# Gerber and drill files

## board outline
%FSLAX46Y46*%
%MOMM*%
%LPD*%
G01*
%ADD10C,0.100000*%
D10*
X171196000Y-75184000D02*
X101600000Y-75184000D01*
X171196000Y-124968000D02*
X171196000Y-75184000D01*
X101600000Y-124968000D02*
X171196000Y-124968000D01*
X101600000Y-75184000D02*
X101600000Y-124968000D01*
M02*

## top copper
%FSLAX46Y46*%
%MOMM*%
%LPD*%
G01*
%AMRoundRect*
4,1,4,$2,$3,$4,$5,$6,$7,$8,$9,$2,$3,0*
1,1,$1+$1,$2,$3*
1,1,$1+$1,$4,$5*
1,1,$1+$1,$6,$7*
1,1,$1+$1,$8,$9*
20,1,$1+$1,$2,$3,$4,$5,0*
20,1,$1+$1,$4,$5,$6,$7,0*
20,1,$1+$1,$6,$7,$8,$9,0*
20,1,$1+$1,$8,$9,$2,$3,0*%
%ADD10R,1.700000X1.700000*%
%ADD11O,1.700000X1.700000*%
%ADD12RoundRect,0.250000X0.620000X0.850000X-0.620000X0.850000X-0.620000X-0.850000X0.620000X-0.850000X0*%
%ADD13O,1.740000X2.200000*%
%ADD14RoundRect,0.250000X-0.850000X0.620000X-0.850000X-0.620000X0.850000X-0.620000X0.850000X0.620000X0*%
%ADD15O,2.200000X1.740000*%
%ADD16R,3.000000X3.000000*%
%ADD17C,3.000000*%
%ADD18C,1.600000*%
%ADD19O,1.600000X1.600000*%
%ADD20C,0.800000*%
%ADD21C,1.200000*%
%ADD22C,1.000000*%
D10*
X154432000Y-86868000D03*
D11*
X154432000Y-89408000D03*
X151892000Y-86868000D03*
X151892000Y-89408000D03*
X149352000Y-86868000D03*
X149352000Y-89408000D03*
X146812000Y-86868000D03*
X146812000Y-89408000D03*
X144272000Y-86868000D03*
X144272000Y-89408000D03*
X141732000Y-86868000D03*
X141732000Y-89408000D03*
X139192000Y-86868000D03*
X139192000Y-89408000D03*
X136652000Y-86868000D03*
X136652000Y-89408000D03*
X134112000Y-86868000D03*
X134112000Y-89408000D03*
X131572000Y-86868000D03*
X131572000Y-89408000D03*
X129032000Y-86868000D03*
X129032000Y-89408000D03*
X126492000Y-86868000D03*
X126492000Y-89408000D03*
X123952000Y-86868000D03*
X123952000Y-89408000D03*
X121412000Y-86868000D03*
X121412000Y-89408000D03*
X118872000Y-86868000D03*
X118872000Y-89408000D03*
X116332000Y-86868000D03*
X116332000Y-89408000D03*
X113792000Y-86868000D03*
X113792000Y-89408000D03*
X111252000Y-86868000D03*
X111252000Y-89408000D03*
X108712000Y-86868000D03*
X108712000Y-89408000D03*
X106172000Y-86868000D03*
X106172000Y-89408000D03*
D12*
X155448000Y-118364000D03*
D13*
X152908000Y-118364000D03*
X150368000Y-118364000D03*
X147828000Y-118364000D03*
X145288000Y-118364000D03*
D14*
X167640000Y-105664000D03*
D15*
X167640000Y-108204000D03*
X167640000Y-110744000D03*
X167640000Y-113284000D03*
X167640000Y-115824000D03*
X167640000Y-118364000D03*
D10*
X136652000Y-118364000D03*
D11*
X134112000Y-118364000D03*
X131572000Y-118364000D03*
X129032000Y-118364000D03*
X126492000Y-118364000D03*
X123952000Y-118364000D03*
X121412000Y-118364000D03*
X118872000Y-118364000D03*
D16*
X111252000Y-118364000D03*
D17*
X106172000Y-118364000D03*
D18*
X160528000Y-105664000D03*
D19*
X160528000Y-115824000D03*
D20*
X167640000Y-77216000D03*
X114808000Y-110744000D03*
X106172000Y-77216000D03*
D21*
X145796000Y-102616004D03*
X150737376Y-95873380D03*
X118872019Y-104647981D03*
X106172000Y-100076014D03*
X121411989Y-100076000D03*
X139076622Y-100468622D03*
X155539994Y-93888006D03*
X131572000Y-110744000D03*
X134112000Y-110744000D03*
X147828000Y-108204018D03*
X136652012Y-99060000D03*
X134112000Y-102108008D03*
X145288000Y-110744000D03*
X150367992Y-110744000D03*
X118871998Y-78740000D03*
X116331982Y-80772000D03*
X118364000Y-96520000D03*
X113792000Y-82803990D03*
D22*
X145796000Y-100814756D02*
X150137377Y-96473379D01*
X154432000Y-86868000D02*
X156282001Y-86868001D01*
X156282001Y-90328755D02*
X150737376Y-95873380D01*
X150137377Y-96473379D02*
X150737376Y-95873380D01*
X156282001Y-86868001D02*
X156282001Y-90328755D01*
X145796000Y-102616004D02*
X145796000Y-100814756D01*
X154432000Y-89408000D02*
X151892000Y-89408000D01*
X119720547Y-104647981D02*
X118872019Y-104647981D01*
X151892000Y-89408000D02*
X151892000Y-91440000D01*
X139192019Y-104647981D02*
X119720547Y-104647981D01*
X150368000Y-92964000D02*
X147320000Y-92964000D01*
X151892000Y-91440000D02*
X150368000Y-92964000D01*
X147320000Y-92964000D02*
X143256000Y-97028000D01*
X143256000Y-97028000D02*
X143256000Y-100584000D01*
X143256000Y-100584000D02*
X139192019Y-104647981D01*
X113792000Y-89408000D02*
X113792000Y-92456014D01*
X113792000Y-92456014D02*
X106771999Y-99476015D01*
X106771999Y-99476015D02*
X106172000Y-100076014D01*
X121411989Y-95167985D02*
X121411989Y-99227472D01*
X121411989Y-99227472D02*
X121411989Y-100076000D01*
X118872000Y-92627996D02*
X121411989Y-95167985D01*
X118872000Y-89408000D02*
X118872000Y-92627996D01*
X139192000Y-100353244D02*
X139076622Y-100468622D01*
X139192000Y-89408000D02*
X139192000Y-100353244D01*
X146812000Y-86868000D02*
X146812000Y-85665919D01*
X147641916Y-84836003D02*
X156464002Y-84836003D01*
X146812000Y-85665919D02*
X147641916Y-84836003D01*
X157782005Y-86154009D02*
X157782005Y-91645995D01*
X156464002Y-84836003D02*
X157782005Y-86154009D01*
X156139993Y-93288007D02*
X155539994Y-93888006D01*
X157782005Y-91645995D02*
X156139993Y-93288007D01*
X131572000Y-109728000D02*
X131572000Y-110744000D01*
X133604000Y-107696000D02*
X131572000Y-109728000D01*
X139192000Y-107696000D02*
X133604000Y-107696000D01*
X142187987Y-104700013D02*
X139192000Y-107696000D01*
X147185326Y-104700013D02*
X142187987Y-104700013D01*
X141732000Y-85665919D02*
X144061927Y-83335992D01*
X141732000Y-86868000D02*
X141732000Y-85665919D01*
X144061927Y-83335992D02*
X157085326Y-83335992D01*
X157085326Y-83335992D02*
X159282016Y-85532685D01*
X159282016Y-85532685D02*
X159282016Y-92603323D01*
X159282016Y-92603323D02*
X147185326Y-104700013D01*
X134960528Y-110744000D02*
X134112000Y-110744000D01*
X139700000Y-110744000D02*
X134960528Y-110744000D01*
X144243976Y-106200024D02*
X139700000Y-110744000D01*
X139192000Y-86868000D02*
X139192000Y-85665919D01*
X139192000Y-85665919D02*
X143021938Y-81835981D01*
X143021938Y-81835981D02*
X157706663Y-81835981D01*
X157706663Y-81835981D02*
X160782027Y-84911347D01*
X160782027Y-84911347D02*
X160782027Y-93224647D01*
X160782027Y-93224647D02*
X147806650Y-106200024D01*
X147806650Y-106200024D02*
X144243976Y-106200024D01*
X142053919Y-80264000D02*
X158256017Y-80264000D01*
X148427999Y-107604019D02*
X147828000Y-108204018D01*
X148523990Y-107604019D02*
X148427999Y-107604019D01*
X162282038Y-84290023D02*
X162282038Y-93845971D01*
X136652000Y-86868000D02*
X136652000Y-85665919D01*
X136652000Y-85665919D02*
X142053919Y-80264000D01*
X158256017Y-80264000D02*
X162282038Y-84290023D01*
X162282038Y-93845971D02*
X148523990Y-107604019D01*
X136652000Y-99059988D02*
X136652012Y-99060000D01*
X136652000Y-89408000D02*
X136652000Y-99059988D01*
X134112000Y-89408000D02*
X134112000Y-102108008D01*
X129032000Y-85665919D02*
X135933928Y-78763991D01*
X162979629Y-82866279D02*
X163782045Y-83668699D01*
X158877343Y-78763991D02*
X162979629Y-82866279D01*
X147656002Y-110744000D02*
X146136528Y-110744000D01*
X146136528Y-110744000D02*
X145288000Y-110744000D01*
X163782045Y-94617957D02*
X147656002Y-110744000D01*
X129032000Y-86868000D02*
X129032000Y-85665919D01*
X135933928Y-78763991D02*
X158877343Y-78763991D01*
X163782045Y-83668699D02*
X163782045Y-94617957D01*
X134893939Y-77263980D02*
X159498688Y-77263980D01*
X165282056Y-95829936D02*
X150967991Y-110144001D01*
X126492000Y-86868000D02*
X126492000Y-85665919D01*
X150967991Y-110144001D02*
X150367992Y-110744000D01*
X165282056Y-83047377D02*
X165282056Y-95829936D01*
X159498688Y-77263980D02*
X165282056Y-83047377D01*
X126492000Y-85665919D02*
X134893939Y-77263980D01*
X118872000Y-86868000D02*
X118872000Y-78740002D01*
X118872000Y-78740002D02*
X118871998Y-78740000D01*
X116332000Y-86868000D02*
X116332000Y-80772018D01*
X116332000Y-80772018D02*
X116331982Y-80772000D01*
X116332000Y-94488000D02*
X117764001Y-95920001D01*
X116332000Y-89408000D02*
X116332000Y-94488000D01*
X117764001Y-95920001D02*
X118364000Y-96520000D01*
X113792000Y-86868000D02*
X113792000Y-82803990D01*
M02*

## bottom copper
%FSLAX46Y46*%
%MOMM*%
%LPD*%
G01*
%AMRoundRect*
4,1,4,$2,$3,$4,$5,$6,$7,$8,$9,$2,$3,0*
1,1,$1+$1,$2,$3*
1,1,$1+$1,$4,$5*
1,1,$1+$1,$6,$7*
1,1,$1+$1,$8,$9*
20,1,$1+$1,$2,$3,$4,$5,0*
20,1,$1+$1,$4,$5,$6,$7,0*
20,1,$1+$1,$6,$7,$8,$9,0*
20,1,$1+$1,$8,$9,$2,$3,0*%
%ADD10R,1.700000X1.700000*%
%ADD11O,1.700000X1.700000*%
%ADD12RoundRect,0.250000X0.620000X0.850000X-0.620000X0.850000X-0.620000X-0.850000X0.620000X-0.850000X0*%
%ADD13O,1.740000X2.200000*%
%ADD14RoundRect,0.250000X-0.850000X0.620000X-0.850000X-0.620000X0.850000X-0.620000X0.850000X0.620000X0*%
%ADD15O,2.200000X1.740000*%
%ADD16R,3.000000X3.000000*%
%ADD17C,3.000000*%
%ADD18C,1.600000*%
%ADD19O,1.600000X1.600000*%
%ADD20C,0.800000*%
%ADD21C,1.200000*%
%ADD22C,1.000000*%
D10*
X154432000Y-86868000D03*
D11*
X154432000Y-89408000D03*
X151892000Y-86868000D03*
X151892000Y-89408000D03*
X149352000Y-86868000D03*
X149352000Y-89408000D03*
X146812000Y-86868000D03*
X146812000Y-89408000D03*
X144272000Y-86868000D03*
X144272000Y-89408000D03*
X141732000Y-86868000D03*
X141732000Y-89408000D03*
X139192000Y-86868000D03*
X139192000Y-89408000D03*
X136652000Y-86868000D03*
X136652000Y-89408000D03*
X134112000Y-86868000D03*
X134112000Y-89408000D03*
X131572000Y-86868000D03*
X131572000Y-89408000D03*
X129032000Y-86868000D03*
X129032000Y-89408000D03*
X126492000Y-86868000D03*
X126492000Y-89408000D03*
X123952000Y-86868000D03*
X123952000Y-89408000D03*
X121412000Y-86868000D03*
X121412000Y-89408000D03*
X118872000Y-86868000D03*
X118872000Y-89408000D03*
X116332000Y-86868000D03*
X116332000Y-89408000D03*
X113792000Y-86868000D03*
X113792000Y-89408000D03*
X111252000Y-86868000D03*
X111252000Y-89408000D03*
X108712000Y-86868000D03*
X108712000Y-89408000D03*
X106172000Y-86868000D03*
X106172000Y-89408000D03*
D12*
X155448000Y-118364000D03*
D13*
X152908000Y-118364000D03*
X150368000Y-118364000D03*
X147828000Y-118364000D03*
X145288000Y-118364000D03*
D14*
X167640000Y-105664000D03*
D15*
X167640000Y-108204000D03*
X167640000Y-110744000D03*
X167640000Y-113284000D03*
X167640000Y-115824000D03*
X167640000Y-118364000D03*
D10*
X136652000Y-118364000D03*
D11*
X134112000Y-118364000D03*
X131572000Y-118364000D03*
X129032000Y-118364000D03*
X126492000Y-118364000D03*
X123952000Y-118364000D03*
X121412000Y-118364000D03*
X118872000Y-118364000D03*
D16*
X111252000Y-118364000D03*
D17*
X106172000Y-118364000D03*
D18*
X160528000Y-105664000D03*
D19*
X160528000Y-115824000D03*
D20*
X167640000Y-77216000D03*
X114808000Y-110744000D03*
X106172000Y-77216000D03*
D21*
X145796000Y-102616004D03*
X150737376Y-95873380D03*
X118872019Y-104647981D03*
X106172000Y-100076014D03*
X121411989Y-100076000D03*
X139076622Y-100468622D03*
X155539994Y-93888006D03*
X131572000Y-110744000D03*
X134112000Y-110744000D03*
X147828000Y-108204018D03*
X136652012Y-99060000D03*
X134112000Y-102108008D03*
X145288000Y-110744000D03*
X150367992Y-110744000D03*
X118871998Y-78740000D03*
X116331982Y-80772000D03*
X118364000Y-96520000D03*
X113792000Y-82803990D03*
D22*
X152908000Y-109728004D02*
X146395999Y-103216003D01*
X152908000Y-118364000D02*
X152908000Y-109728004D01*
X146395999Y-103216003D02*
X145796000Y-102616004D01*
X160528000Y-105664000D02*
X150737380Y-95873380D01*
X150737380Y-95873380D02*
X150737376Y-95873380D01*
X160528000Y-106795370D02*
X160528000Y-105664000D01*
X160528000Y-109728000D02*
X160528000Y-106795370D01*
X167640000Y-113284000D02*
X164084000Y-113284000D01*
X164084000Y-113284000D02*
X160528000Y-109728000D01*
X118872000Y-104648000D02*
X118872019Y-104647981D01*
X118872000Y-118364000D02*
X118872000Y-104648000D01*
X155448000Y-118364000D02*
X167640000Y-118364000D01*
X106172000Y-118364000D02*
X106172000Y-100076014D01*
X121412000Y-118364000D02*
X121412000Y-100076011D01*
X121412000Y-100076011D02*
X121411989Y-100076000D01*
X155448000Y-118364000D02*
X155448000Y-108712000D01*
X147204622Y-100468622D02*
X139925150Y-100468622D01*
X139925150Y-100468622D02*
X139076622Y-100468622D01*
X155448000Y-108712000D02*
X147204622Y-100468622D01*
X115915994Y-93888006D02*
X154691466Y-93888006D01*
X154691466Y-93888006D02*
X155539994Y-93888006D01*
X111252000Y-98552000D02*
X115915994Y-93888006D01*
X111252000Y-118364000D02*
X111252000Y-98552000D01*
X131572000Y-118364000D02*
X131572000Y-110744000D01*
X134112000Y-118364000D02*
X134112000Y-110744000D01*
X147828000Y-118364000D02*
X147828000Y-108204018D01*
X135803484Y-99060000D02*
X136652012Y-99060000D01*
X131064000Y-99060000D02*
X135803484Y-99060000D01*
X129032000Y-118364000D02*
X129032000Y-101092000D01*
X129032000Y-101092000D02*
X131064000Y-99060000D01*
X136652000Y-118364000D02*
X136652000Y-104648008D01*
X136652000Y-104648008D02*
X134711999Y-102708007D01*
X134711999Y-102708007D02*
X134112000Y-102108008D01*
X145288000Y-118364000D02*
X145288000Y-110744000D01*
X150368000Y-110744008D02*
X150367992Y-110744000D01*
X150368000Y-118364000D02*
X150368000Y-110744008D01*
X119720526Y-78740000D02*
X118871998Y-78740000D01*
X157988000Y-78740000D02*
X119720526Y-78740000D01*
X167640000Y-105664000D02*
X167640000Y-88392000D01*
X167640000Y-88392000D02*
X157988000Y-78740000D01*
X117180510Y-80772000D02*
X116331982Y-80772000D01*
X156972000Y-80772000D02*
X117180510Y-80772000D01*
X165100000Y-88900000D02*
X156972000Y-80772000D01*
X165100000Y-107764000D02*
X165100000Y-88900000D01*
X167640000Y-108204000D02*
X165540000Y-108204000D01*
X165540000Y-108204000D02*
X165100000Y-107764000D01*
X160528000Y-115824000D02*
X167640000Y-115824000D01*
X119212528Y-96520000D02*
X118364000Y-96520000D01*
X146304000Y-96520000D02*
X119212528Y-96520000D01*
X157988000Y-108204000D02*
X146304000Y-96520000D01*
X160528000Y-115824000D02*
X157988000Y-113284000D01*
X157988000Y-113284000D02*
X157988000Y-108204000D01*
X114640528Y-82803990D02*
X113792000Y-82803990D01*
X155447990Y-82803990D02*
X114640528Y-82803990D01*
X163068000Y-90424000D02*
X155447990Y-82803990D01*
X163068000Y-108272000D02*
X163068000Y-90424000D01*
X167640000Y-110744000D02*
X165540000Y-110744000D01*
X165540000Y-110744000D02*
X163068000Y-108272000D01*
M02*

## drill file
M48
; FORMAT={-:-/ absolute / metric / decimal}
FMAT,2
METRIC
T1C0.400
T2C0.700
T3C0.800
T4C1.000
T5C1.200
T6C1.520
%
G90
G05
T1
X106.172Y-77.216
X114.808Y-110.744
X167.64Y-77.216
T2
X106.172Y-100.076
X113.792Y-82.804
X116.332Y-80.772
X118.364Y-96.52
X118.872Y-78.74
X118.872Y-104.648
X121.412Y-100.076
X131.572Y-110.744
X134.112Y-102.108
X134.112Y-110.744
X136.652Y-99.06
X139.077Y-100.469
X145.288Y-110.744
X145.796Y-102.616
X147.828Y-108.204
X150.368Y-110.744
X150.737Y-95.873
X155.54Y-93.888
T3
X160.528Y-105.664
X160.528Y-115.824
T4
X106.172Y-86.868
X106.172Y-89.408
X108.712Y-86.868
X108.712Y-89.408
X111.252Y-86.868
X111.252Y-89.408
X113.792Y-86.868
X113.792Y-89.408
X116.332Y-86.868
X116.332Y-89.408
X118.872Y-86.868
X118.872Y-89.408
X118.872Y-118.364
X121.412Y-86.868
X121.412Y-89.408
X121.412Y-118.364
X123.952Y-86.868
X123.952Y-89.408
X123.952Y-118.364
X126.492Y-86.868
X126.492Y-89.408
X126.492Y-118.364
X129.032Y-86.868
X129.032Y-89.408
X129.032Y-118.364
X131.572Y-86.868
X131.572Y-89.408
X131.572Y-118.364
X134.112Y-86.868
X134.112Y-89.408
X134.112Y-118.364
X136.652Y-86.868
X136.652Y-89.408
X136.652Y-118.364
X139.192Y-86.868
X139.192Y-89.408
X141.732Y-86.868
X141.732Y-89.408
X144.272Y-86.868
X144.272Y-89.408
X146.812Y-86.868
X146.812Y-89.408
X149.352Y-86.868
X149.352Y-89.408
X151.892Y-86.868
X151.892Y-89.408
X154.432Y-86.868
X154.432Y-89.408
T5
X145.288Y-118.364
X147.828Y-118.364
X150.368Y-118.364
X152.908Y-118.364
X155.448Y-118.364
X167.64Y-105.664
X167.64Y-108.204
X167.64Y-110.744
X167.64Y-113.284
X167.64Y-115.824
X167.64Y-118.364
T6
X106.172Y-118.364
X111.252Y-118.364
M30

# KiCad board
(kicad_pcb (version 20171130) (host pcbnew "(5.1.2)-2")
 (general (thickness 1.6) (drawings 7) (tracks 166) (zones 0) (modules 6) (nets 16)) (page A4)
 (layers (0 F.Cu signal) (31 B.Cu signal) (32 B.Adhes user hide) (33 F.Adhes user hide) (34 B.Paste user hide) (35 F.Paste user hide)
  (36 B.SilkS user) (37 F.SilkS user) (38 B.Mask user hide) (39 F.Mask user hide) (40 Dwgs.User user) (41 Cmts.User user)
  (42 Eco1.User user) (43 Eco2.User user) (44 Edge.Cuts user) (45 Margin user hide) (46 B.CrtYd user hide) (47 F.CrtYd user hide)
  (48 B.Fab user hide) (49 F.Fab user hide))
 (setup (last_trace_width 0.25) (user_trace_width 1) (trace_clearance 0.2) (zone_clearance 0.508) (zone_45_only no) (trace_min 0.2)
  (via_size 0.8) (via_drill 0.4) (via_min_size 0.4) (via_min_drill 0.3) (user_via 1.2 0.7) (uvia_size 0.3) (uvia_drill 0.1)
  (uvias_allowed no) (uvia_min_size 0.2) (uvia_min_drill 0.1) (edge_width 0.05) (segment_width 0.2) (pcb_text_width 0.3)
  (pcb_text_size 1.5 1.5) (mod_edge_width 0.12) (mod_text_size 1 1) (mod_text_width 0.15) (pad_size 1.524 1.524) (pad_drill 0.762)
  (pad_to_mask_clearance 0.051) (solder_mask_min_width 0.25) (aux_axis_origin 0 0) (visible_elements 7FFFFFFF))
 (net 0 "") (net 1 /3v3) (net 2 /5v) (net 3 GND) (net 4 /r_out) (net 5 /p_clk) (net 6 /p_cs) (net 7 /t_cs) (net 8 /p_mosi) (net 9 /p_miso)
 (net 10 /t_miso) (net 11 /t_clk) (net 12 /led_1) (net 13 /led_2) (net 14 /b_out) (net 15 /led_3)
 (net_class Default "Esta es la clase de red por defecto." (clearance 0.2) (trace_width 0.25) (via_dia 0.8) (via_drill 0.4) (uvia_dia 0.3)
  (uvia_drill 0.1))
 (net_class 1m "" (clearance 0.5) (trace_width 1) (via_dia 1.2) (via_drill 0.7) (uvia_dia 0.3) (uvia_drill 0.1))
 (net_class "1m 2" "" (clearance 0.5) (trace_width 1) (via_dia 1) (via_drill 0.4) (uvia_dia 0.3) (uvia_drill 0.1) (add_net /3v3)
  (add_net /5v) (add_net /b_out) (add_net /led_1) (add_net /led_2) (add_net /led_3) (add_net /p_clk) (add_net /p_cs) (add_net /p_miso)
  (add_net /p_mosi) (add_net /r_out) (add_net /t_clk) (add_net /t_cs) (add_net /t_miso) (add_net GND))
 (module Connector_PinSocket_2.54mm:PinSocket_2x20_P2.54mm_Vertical (layer B.Cu) (at 154.432 86.868 90)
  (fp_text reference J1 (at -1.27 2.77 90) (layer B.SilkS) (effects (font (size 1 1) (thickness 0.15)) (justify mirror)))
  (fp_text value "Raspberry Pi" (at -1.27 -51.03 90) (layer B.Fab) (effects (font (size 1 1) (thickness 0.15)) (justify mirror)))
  (pad 1 thru_hole rect (at 0 0 90) (size 1.7 1.7) (drill 1) (layers *.Cu *.Mask) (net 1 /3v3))
  (pad 2 thru_hole oval (at -2.54 0 90) (size 1.7 1.7) (drill 1) (layers *.Cu *.Mask) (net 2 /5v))
  (pad 3 thru_hole oval (at 0 -2.54 90) (size 1.7 1.7) (drill 1) (layers *.Cu *.Mask))
  (pad 4 thru_hole oval (at -2.54 -2.54 90) (size 1.7 1.7) (drill 1) (layers *.Cu *.Mask) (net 2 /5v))
  (pad 5 thru_hole oval (at 0 -5.08 90) (size 1.7 1.7) (drill 1) (layers *.Cu *.Mask))
  (pad 6 thru_hole oval (at -2.54 -5.08 90) (size 1.7 1.7) (drill 1) (layers *.Cu *.Mask) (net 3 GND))
  (pad 7 thru_hole oval (at 0 -7.62 90) (size 1.7 1.7) (drill 1) (layers *.Cu *.Mask) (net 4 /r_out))
  (pad 8 thru_hole oval (at -2.54 -7.62 90) (size 1.7 1.7) (drill 1) (layers *.Cu *.Mask))
  (pad 9 thru_hole oval (at 0 -10.16 90) (size 1.7 1.7) (drill 1) (layers *.Cu *.Mask))
  (pad 10 thru_hole oval (at -2.54 -10.16 90) (size 1.7 1.7) (drill 1) (layers *.Cu *.Mask))
  (pad 11 thru_hole oval (at 0 -12.7 90) (size 1.7 1.7) (drill 1) (layers *.Cu *.Mask) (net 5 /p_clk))
  (pad 12 thru_hole oval (at -2.54 -12.7 90) (size 1.7 1.7) (drill 1) (layers *.Cu *.Mask))
  (pad 13 thru_hole oval (at 0 -15.24 90) (size 1.7 1.7) (drill 1) (layers *.Cu *.Mask) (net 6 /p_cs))
  (pad 14 thru_hole oval (at -2.54 -15.24 90) (size 1.7 1.7) (drill 1) (layers *.Cu *.Mask) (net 3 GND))
  (pad 15 thru_hole oval (at 0 -17.78 90) (size 1.7 1.7) (drill 1) (layers *.Cu *.Mask) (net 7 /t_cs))
  (pad 16 thru_hole oval (at -2.54 -17.78 90) (size 1.7 1.7) (drill 1) (layers *.Cu *.Mask) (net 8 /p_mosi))
  (pad 17 thru_hole oval (at 0 -20.32 90) (size 1.7 1.7) (drill 1) (layers *.Cu *.Mask))
  (pad 18 thru_hole oval (at -2.54 -20.32 90) (size 1.7 1.7) (drill 1) (layers *.Cu *.Mask) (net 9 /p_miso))
  (pad 19 thru_hole oval (at 0 -22.86 90) (size 1.7 1.7) (drill 1) (layers *.Cu *.Mask))
  (pad 20 thru_hole oval (at -2.54 -22.86 90) (size 1.7 1.7) (drill 1) (layers *.Cu *.Mask) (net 3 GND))
  (pad 21 thru_hole oval (at 0 -25.4 90) (size 1.7 1.7) (drill 1) (layers *.Cu *.Mask) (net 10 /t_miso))
  (pad 22 thru_hole oval (at -2.54 -25.4 90) (size 1.7 1.7) (drill 1) (layers *.Cu *.Mask))
  (pad 23 thru_hole oval (at 0 -27.94 90) (size 1.7 1.7) (drill 1) (layers *.Cu *.Mask) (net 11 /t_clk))
  (pad 24 thru_hole oval (at -2.54 -27.94 90) (size 1.7 1.7) (drill 1) (layers *.Cu *.Mask))
  (pad 25 thru_hole oval (at 0 -30.48 90) (size 1.7 1.7) (drill 1) (layers *.Cu *.Mask))
  (pad 26 thru_hole oval (at -2.54 -30.48 90) (size 1.7 1.7) (drill 1) (layers *.Cu *.Mask))
  (pad 27 thru_hole oval (at 0 -33.02 90) (size 1.7 1.7) (drill 1) (layers *.Cu *.Mask))
  (pad 28 thru_hole oval (at -2.54 -33.02 90) (size 1.7 1.7) (drill 1) (layers *.Cu *.Mask))
  (pad 29 thru_hole oval (at 0 -35.56 90) (size 1.7 1.7) (drill 1) (layers *.Cu *.Mask) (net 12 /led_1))
  (pad 30 thru_hole oval (at -2.54 -35.56 90) (size 1.7 1.7) (drill 1) (layers *.Cu *.Mask) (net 3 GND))
  (pad 31 thru_hole oval (at 0 -38.1 90) (size 1.7 1.7) (drill 1) (layers *.Cu *.Mask) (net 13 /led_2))
  (pad 32 thru_hole oval (at -2.54 -38.1 90) (size 1.7 1.7) (drill 1) (layers *.Cu *.Mask) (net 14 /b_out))
  (pad 33 thru_hole oval (at 0 -40.64 90) (size 1.7 1.7) (drill 1) (layers *.Cu *.Mask) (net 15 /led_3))
  (pad 34 thru_hole oval (at -2.54 -40.64 90) (size 1.7 1.7) (drill 1) (layers *.Cu *.Mask) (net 3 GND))
  (pad 35 thru_hole oval (at 0 -43.18 90) (size 1.7 1.7) (drill 1) (layers *.Cu *.Mask))
  (pad 36 thru_hole oval (at -2.54 -43.18 90) (size 1.7 1.7) (drill 1) (layers *.Cu *.Mask))
  (pad 37 thru_hole oval (at 0 -45.72 90) (size 1.7 1.7) (drill 1) (layers *.Cu *.Mask))
  (pad 38 thru_hole oval (at -2.54 -45.72 90) (size 1.7 1.7) (drill 1) (layers *.Cu *.Mask))
  (pad 39 thru_hole oval (at 0 -48.26 90) (size 1.7 1.7) (drill 1) (layers *.Cu *.Mask))
  (pad 40 thru_hole oval (at -2.54 -48.26 90) (size 1.7 1.7) (drill 1) (layers *.Cu *.Mask)))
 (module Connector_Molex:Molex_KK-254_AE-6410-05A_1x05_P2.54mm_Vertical (layer F.Cu) (at 155.448 118.364 180)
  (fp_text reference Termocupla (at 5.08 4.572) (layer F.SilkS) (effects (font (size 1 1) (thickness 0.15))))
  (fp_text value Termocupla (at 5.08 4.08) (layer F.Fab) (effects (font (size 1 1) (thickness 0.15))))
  (pad 1 thru_hole roundrect (at 0 0 180) (size 1.74 2.2) (drill 1.2) (layers *.Cu *.Mask) (roundrect_rratio 0.143678) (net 3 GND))
  (pad 2 thru_hole oval (at 2.54 0 180) (size 1.74 2.2) (drill 1.2) (layers *.Cu *.Mask) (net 1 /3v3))
  (pad 3 thru_hole oval (at 5.08 0 180) (size 1.74 2.2) (drill 1.2) (layers *.Cu *.Mask) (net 11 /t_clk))
  (pad 4 thru_hole oval (at 7.62 0 180) (size 1.74 2.2) (drill 1.2) (layers *.Cu *.Mask) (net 7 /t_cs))
  (pad 5 thru_hole oval (at 10.16 0 180) (size 1.74 2.2) (drill 1.2) (layers *.Cu *.Mask) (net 10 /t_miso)))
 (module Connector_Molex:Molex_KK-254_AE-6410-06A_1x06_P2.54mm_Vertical (layer F.Cu) (at 167.64 105.664 270)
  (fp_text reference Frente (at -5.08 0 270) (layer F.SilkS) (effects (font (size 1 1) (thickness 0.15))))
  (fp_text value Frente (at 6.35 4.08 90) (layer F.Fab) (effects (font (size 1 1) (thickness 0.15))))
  (pad 1 thru_hole roundrect (at 0 0 270) (size 1.74 2.2) (drill 1.2) (layers *.Cu *.Mask) (roundrect_rratio 0.143678) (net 12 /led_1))
  (pad 2 thru_hole oval (at 2.54 0 270) (size 1.74 2.2) (drill 1.2) (layers *.Cu *.Mask) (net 13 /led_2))
  (pad 3 thru_hole oval (at 5.08 0 270) (size 1.74 2.2) (drill 1.2) (layers *.Cu *.Mask) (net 15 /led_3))
  (pad 4 thru_hole oval (at 7.62 0 270) (size 1.74 2.2) (drill 1.2) (layers *.Cu *.Mask) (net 1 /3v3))
  (pad 5 thru_hole oval (at 10.16 0 270) (size 1.74 2.2) (drill 1.2) (layers *.Cu *.Mask) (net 14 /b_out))
  (pad 6 thru_hole oval (at 12.7 0 270) (size 1.74 2.2) (drill 1.2) (layers *.Cu *.Mask) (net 3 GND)))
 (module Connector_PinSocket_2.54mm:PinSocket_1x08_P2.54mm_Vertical (layer F.Cu) (at 136.652 118.364 270)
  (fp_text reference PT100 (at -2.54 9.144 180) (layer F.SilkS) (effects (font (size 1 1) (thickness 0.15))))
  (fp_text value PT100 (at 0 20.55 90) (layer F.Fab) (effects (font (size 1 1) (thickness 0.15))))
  (pad 1 thru_hole rect (at 0 0 270) (size 1.7 1.7) (drill 1) (layers *.Cu *.Mask) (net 9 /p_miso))
  (pad 2 thru_hole oval (at 0 2.54 270) (size 1.7 1.7) (drill 1) (layers *.Cu *.Mask) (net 6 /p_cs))
  (pad 3 thru_hole oval (at 0 5.08 270) (size 1.7 1.7) (drill 1) (layers *.Cu *.Mask) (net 5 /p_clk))
  (pad 4 thru_hole oval (at 0 7.62 270) (size 1.7 1.7) (drill 1) (layers *.Cu *.Mask) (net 8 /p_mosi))
  (pad 5 thru_hole oval (at 0 10.16 270) (size 1.7 1.7) (drill 1) (layers *.Cu *.Mask))
  (pad 6 thru_hole oval (at 0 12.7 270) (size 1.7 1.7) (drill 1) (layers *.Cu *.Mask))
  (pad 7 thru_hole oval (at 0 15.24 270) (size 1.7 1.7) (drill 1) (layers *.Cu *.Mask) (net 3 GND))
  (pad 8 thru_hole oval (at 0 17.78 270) (size 1.7 1.7) (drill 1) (layers *.Cu *.Mask) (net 2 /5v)))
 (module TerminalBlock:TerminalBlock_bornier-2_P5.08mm (layer F.Cu) (at 111.252 118.364 180)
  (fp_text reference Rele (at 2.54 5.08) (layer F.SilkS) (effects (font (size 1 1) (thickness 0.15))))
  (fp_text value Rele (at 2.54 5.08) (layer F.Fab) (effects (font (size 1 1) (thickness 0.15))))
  (pad 1 thru_hole rect (at 0 0 180) (size 3 3) (drill 1.52) (layers *.Cu *.Mask) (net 4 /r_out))
  (pad 2 thru_hole circle (at 5.08 0 180) (size 3 3) (drill 1.52) (layers *.Cu *.Mask) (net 3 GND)))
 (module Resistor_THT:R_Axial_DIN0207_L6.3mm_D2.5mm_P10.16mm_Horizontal (layer F.Cu) (at 160.528 105.664 270)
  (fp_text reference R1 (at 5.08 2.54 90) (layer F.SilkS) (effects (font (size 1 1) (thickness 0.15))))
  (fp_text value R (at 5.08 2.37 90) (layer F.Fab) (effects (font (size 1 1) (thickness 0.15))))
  (pad 1 thru_hole circle (at 0 0 270) (size 1.6 1.6) (drill 0.8) (layers *.Cu *.Mask) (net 1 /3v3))
  (pad 2 thru_hole oval (at 10.16 0 270) (size 1.6 1.6) (drill 0.8) (layers *.Cu *.Mask) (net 14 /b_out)))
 (gr_line (start 171.196 75.184) (end 101.6 75.184) (layer Edge.Cuts) (width 0.1))
 (gr_line (start 171.196 124.968) (end 171.196 75.184) (layer Edge.Cuts) (width 0.1))
 (gr_line (start 101.6 124.968) (end 171.196 124.968) (layer Edge.Cuts) (width 0.1))
 (gr_line (start 101.6 75.184) (end 101.6 124.968) (layer Edge.Cuts) (width 0.1))
 (via (at 167.64 77.216) (size 0.8) (drill 0.4) (layers F.Cu B.Cu) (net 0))
 (via (at 114.808 110.744) (size 0.8) (drill 0.4) (layers F.Cu B.Cu) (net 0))
 (via (at 106.172 77.216) (size 0.8) (drill 0.4) (layers F.Cu B.Cu) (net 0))
 (segment (start 152.908 109.728004) (end 146.395999 103.216003) (width 1) (layer B.Cu) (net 1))
 (segment (start 152.908 118.364) (end 152.908 109.728004) (width 1) (layer B.Cu) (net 1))
 (via (at 145.796 102.616004) (size 1.2) (drill 0.7) (layers F.Cu B.Cu) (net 1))
 (segment (start 146.395999 103.216003) (end 145.796 102.616004) (width 1) (layer B.Cu) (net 1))
 (via (at 150.737376 95.87338) (size 1.2) (drill 0.7) (layers F.Cu B.Cu) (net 1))
 (segment (start 145.796 100.814756) (end 150.137377 96.473379) (width 1) (layer F.Cu) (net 1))
 (segment (start 160.528 105.664) (end 150.73738 95.87338) (width 1) (layer B.Cu) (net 1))
 (segment (start 154.432 86.868) (end 156.282001 86.868001) (width 1) (layer F.Cu) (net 1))
 (segment (start 156.282001 90.328755) (end 150.737376 95.87338) (width 1) (layer F.Cu) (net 1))
 (segment (start 150.137377 96.473379) (end 150.737376 95.87338) (width 1) (layer F.Cu) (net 1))
 (segment (start 156.282001 86.868001) (end 156.282001 90.328755) (width 1) (layer F.Cu) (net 1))
 (segment (start 145.796 102.616004) (end 145.796 100.814756) (width 1) (layer F.Cu) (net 1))
 (segment (start 150.73738 95.87338) (end 150.737376 95.87338) (width 1) (layer B.Cu) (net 1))
 (segment (start 160.528 106.79537) (end 160.528 105.664) (width 1) (layer B.Cu) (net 1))
 (segment (start 160.528 109.728) (end 160.528 106.79537) (width 1) (layer B.Cu) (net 1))
 (segment (start 167.64 113.284) (end 164.084 113.284) (width 1) (layer B.Cu) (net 1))
 (segment (start 164.084 113.284) (end 160.528 109.728) (width 1) (layer B.Cu) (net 1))
 (segment (start 154.432 89.408) (end 151.892 89.408) (width 1) (layer F.Cu) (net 2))
 (segment (start 118.872 104.648) (end 118.872019 104.647981) (width 1) (layer B.Cu) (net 2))
 (segment (start 118.872 118.364) (end 118.872 104.648) (width 1) (layer B.Cu) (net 2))
 (via (at 118.872019 104.647981) (size 1.2) (drill 0.7) (layers F.Cu B.Cu) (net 2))
 (segment (start 119.720547 104.647981) (end 118.872019 104.647981) (width 1) (layer F.Cu) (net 2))
 (segment (start 151.892 89.408) (end 151.892 91.44) (width 1) (layer F.Cu) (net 2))
 (segment (start 139.192019 104.647981) (end 119.720547 104.647981) (width 1) (layer F.Cu) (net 2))
 (segment (start 150.368 92.964) (end 147.32 92.964) (width 1) (layer F.Cu) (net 2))
 (segment (start 151.892 91.44) (end 150.368 92.964) (width 1) (layer F.Cu) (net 2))
 (segment (start 147.32 92.964) (end 143.256 97.028) (width 1) (layer F.Cu) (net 2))
 (segment (start 143.256 97.028) (end 143.256 100.584) (width 1) (layer F.Cu) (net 2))
 (segment (start 143.256 100.584) (end 139.192019 104.647981) (width 1) (layer F.Cu) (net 2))
 (segment (start 155.448 118.364) (end 167.64 118.364) (width 1) (layer B.Cu) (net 3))
 (via (at 106.172 100.076014) (size 1.2) (drill 0.7) (layers F.Cu B.Cu) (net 3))
 (segment (start 106.172 118.364) (end 106.172 100.076014) (width 1) (layer B.Cu) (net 3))
 (segment (start 113.792 89.408) (end 113.792 92.456014) (width 1) (layer F.Cu) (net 3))
 (segment (start 113.792 92.456014) (end 106.771999 99.476015) (width 1) (layer F.Cu) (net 3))
 (segment (start 106.771999 99.476015) (end 106.172 100.076014) (width 1) (layer F.Cu) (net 3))
 (via (at 121.411989 100.076) (size 1.2) (drill 0.7) (layers F.Cu B.Cu) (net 3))
 (segment (start 121.411989 95.167985) (end 121.411989 99.227472) (width 1) (layer F.Cu) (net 3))
 (segment (start 121.411989 99.227472) (end 121.411989 100.076) (width 1) (layer F.Cu) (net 3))
 (segment (start 118.872 92.627996) (end 121.411989 95.167985) (width 1) (layer F.Cu) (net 3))
 (segment (start 118.872 89.408) (end 118.872 92.627996) (width 1) (layer F.Cu) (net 3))
 (segment (start 121.412 118.364) (end 121.412 100.076011) (width 1) (layer B.Cu) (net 3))
 (segment (start 121.412 100.076011) (end 121.411989 100.076) (width 1) (layer B.Cu) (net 3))
 (via (at 139.076622 100.468622) (size 1.2) (drill 0.7) (layers F.Cu B.Cu) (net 3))
 (segment (start 155.448 118.364) (end 155.448 108.712) (width 1) (layer B.Cu) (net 3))
 (segment (start 147.204622 100.468622) (end 139.92515 100.468622) (width 1) (layer B.Cu) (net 3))
 (segment (start 139.92515 100.468622) (end 139.076622 100.468622) (width 1) (layer B.Cu) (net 3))
 (segment (start 139.192 100.353244) (end 139.076622 100.468622) (width 1) (layer F.Cu) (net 3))
 (segment (start 139.192 89.408) (end 139.192 100.353244) (width 1) (layer F.Cu) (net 3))
 (segment (start 155.448 108.712) (end 147.204622 100.468622) (width 1) (layer B.Cu) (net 3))
 (via (at 155.539994 93.888006) (size 1.2) (drill 0.7) (layers F.Cu B.Cu) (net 4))
 (segment (start 146.812 86.868) (end 146.812 85.665919) (width 1) (layer F.Cu) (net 4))
 (segment (start 147.641916 84.836003) (end 156.464002 84.836003) (width 1) (layer F.Cu) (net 4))
 (segment (start 146.812 85.665919) (end 147.641916 84.836003) (width 1) (layer F.Cu) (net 4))
 (segment (start 157.782005 86.154009) (end 157.782005 91.645995) (width 1) (layer F.Cu) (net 4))
 (segment (start 156.464002 84.836003) (end 157.782005 86.154009) (width 1) (layer F.Cu) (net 4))
 (segment (start 156.139993 93.288007) (end 155.539994 93.888006) (width 1) (layer F.Cu) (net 4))
 (segment (start 157.782005 91.645995) (end 156.139993 93.288007) (width 1) (layer F.Cu) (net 4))
 (segment (start 115.915994 93.888006) (end 154.691466 93.888006) (width 1) (layer B.Cu) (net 4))
 (segment (start 154.691466 93.888006) (end 155.539994 93.888006) (width 1) (layer B.Cu) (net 4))
 (segment (start 111.252 98.552) (end 115.915994 93.888006) (width 1) (layer B.Cu) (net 4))
 (segment (start 111.252 118.364) (end 111.252 98.552) (width 1) (layer B.Cu) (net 4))
 (segment (start 131.572 118.364) (end 131.572 110.744) (width 1) (layer B.Cu) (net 5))
 (via (at 131.572 110.744) (size 1.2) (drill 0.7) (layers F.Cu B.Cu) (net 5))
 (segment (start 131.572 109.728) (end 131.572 110.744) (width 1) (layer F.Cu) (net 5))
 (segment (start 133.604 107.696) (end 131.572 109.728) (width 1) (layer F.Cu) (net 5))
 (segment (start 139.192 107.696) (end 133.604 107.696) (width 1) (layer F.Cu) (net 5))
 (segment (start 142.187987 104.700013) (end 139.192 107.696) (width 1) (layer F.Cu) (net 5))
 (segment (start 147.185326 104.700013) (end 142.187987 104.700013) (width 1) (layer F.Cu) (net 5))
 (segment (start 141.732 85.665919) (end 144.061927 83.335992) (width 1) (layer F.Cu) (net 5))
 (segment (start 141.732 86.868) (end 141.732 85.665919) (width 1) (layer F.Cu) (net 5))
 (segment (start 144.061927 83.335992) (end 157.085326 83.335992) (width 1) (layer F.Cu) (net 5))
 (segment (start 157.085326 83.335992) (end 159.282016 85.532685) (width 1) (layer F.Cu) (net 5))
 (segment (start 159.282016 85.532685) (end 159.282016 92.603323) (width 1) (layer F.Cu) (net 5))
 (segment (start 159.282016 92.603323) (end 147.185326 104.700013) (width 1) (layer F.Cu) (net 5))
 (segment (start 134.112 118.364) (end 134.112 110.744) (width 1) (layer B.Cu) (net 6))
 (via (at 134.112 110.744) (size 1.2) (drill 0.7) (layers F.Cu B.Cu) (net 6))
 (segment (start 134.960528 110.744) (end 134.112 110.744) (width 1) (layer F.Cu) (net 6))
 (segment (start 139.7 110.744) (end 134.960528 110.744) (width 1) (layer F.Cu) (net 6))
 (segment (start 144.243976 106.200024) (end 139.7 110.744) (width 1) (layer F.Cu) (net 6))
 (segment (start 139.192 86.868) (end 139.192 85.665919) (width 1) (layer F.Cu) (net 6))
 (segment (start 139.192 85.665919) (end 143.021938 81.835981) (width 1) (layer F.Cu) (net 6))
 (segment (start 143.021938 81.835981) (end 157.706663 81.835981) (width 1) (layer F.Cu) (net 6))
 (segment (start 157.706663 81.835981) (end 160.782027 84.911347) (width 1) (layer F.Cu) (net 6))
 (segment (start 160.782027 84.911347) (end 160.782027 93.224647) (width 1) (layer F.Cu) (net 6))
 (segment (start 160.782027 93.224647) (end 147.80665 106.200024) (width 1) (layer F.Cu) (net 6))
 (segment (start 147.80665 106.200024) (end 144.243976 106.200024) (width 1) (layer F.Cu) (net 6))
 (segment (start 147.828 118.364) (end 147.828 108.204018) (width 1) (layer B.Cu) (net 7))
 (via (at 147.828 108.204018) (size 1.2) (drill 0.7) (layers F.Cu B.Cu) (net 7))
 (segment (start 142.053919 80.264) (end 158.256017 80.264) (width 1) (layer F.Cu) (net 7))
 (segment (start 148.427999 107.604019) (end 147.828 108.204018) (width 1) (layer F.Cu) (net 7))
 (segment (start 148.52399 107.604019) (end 148.427999 107.604019) (width 1) (layer F.Cu) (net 7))
 (segment (start 162.282038 84.290023) (end 162.282038 93.845971) (width 1) (layer F.Cu) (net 7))
 (segment (start 136.652 86.868) (end 136.652 85.665919) (width 1) (layer F.Cu) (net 7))
 (segment (start 136.652 85.665919) (end 142.053919 80.264) (width 1) (layer F.Cu) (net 7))
 (segment (start 158.256017 80.264) (end 162.282038 84.290023) (width 1) (layer F.Cu) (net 7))
 (segment (start 162.282038 93.845971) (end 148.52399 107.604019) (width 1) (layer F.Cu) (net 7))
 (via (at 136.652012 99.06) (size 1.2) (drill 0.7) (layers F.Cu B.Cu) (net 8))
 (segment (start 136.652 99.059988) (end 136.652012 99.06) (width 1) (layer F.Cu) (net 8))
 (segment (start 136.652 89.408) (end 136.652 99.059988) (width 1) (layer F.Cu) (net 8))
 (segment (start 135.803484 99.06) (end 136.652012 99.06) (width 1) (layer B.Cu) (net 8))
 (segment (start 131.064 99.06) (end 135.803484 99.06) (width 1) (layer B.Cu) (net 8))
 (segment (start 129.032 118.364) (end 129.032 101.092) (width 1) (layer B.Cu) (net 8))
 (segment (start 129.032 101.092) (end 131.064 99.06) (width 1) (layer B.Cu) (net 8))
 (via (at 134.112 102.108008) (size 1.2) (drill 0.7) (layers F.Cu B.Cu) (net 9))
 (segment (start 134.112 89.408) (end 134.112 102.108008) (width 1) (layer F.Cu) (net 9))
 (segment (start 136.652 118.364) (end 136.652 104.648008) (width 1) (layer B.Cu) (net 9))
 (segment (start 136.652 104.648008) (end 134.711999 102.708007) (width 1) (layer B.Cu) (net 9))
 (segment (start 134.711999 102.708007) (end 134.112 102.108008) (width 1) (layer B.Cu) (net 9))
 (segment (start 145.288 118.364) (end 145.288 110.744) (width 1) (layer B.Cu) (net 10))
 (via (at 145.288 110.744) (size 1.2) (drill 0.7) (layers F.Cu B.Cu) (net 10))
 (segment (start 129.032 85.665919) (end 135.933928 78.763991) (width 1) (layer F.Cu) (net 10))
 (segment (start 162.979629 82.866279) (end 163.782045 83.668699) (width 1) (layer F.Cu) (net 10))
 (segment (start 158.877343 78.763991) (end 162.979629 82.866279) (width 1) (layer F.Cu) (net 10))
 (segment (start 147.656002 110.744) (end 146.136528 110.744) (width 1) (layer F.Cu) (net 10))
 (segment (start 146.136528 110.744) (end 145.288 110.744) (width 1) (layer F.Cu) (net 10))
 (segment (start 163.782045 94.617957) (end 147.656002 110.744) (width 1) (layer F.Cu) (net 10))
 (segment (start 129.032 86.868) (end 129.032 85.665919) (width 1) (layer F.Cu) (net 10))
 (segment (start 135.933928 78.763991) (end 158.877343 78.763991) (width 1) (layer F.Cu) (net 10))
 (segment (start 163.782045 83.668699) (end 163.782045 94.617957) (width 1) (layer F.Cu) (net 10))
 (segment (start 150.368 110.744008) (end 150.367992 110.744) (width 1) (layer B.Cu) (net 11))
 (segment (start 134.893939 77.26398) (end 159.498688 77.26398) (width 1) (layer F.Cu) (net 11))
 (segment (start 165.282056 95.829936) (end 150.967991 110.144001) (width 1) (layer F.Cu) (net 11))
 (via (at 150.367992 110.744) (size 1.2) (drill 0.7) (layers F.Cu B.Cu) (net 11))
 (segment (start 150.368 118.364) (end 150.368 110.744008) (width 1) (layer B.Cu) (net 11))
 (segment (start 126.492 86.868) (end 126.492 85.665919) (width 1) (layer F.Cu) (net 11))
 (segment (start 150.967991 110.144001) (end 150.367992 110.744) (width 1) (layer F.Cu) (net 11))
 (segment (start 165.282056 83.047377) (end 165.282056 95.829936) (width 1) (layer F.Cu) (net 11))
 (segment (start 159.498688 77.26398) (end 165.282056 83.047377) (width 1) (layer F.Cu) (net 11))
 (segment (start 126.492 85.665919) (end 134.893939 77.26398) (width 1) (layer F.Cu) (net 11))
 (via (at 118.871998 78.74) (size 1.2) (drill 0.7) (layers F.Cu B.Cu) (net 12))
 (segment (start 118.872 86.868) (end 118.872 78.740002) (width 1) (layer F.Cu) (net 12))
 (segment (start 118.872 78.740002) (end 118.871998 78.74) (width 1) (layer F.Cu) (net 12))
 (segment (start 119.720526 78.74) (end 118.871998 78.74) (width 1) (layer B.Cu) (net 12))
 (segment (start 157.988 78.74) (end 119.720526 78.74) (width 1) (layer B.Cu) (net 12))
 (segment (start 167.64 105.664) (end 167.64 88.392) (width 1) (layer B.Cu) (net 12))
 (segment (start 167.64 88.392) (end 157.988 78.74) (width 1) (layer B.Cu) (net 12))
 (via (at 116.331982 80.772) (size 1.2) (drill 0.7) (layers F.Cu B.Cu) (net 13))
 (segment (start 116.332 86.868) (end 116.332 80.772018) (width 1) (layer F.Cu) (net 13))
 (segment (start 116.332 80.772018) (end 116.331982 80.772) (width 1) (layer F.Cu) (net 13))
 (segment (start 117.18051 80.772) (end 116.331982 80.772) (width 1) (layer B.Cu) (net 13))
 (segment (start 156.972 80.772) (end 117.18051 80.772) (width 1) (layer B.Cu) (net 13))
 (segment (start 165.1 88.9) (end 156.972 80.772) (width 1) (layer B.Cu) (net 13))
 (segment (start 165.1 107.764) (end 165.1 88.9) (width 1) (layer B.Cu) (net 13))
 (segment (start 167.64 108.204) (end 165.54 108.204) (width 1) (layer B.Cu) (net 13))
 (segment (start 165.54 108.204) (end 165.1 107.764) (width 1) (layer B.Cu) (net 13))
 (segment (start 160.528 115.824) (end 167.64 115.824) (width 1) (layer B.Cu) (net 14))
 (segment (start 116.332 94.488) (end 117.764001 95.920001) (width 1) (layer F.Cu) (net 14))
 (segment (start 116.332 89.408) (end 116.332 94.488) (width 1) (layer F.Cu) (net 14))
 (segment (start 117.764001 95.920001) (end 118.364 96.52) (width 1) (layer F.Cu) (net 14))
 (via (at 118.364 96.52) (size 1.2) (drill 0.7) (layers F.Cu B.Cu) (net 14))
 (segment (start 119.212528 96.52) (end 118.364 96.52) (width 1) (layer B.Cu) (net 14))
 (segment (start 146.304 96.52) (end 119.212528 96.52) (width 1) (layer B.Cu) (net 14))
 (segment (start 157.988 108.204) (end 146.304 96.52) (width 1) (layer B.Cu) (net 14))
 (segment (start 160.528 115.824) (end 157.988 113.284) (width 1) (layer B.Cu) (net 14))
 (segment (start 157.988 113.284) (end 157.988 108.204) (width 1) (layer B.Cu) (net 14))
 (via (at 113.792 82.80399) (size 1.2) (drill 0.7) (layers F.Cu B.Cu) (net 15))
 (segment (start 113.792 86.868) (end 113.792 82.80399) (width 1) (layer F.Cu) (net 15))
 (segment (start 114.640528 82.80399) (end 113.792 82.80399) (width 1) (layer B.Cu) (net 15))
 (segment (start 155.44799 82.80399) (end 114.640528 82.80399) (width 1) (layer B.Cu) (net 15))
 (segment (start 163.068 90.424) (end 155.44799 82.80399) (width 1) (layer B.Cu) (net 15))
 (segment (start 163.068 108.272) (end 163.068 90.424) (width 1) (layer B.Cu) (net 15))
 (segment (start 167.64 110.744) (end 165.54 110.744) (width 1) (layer B.Cu) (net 15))
 (segment (start 165.54 110.744) (end 163.068 108.272) (width 1) (layer B.Cu) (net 15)))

